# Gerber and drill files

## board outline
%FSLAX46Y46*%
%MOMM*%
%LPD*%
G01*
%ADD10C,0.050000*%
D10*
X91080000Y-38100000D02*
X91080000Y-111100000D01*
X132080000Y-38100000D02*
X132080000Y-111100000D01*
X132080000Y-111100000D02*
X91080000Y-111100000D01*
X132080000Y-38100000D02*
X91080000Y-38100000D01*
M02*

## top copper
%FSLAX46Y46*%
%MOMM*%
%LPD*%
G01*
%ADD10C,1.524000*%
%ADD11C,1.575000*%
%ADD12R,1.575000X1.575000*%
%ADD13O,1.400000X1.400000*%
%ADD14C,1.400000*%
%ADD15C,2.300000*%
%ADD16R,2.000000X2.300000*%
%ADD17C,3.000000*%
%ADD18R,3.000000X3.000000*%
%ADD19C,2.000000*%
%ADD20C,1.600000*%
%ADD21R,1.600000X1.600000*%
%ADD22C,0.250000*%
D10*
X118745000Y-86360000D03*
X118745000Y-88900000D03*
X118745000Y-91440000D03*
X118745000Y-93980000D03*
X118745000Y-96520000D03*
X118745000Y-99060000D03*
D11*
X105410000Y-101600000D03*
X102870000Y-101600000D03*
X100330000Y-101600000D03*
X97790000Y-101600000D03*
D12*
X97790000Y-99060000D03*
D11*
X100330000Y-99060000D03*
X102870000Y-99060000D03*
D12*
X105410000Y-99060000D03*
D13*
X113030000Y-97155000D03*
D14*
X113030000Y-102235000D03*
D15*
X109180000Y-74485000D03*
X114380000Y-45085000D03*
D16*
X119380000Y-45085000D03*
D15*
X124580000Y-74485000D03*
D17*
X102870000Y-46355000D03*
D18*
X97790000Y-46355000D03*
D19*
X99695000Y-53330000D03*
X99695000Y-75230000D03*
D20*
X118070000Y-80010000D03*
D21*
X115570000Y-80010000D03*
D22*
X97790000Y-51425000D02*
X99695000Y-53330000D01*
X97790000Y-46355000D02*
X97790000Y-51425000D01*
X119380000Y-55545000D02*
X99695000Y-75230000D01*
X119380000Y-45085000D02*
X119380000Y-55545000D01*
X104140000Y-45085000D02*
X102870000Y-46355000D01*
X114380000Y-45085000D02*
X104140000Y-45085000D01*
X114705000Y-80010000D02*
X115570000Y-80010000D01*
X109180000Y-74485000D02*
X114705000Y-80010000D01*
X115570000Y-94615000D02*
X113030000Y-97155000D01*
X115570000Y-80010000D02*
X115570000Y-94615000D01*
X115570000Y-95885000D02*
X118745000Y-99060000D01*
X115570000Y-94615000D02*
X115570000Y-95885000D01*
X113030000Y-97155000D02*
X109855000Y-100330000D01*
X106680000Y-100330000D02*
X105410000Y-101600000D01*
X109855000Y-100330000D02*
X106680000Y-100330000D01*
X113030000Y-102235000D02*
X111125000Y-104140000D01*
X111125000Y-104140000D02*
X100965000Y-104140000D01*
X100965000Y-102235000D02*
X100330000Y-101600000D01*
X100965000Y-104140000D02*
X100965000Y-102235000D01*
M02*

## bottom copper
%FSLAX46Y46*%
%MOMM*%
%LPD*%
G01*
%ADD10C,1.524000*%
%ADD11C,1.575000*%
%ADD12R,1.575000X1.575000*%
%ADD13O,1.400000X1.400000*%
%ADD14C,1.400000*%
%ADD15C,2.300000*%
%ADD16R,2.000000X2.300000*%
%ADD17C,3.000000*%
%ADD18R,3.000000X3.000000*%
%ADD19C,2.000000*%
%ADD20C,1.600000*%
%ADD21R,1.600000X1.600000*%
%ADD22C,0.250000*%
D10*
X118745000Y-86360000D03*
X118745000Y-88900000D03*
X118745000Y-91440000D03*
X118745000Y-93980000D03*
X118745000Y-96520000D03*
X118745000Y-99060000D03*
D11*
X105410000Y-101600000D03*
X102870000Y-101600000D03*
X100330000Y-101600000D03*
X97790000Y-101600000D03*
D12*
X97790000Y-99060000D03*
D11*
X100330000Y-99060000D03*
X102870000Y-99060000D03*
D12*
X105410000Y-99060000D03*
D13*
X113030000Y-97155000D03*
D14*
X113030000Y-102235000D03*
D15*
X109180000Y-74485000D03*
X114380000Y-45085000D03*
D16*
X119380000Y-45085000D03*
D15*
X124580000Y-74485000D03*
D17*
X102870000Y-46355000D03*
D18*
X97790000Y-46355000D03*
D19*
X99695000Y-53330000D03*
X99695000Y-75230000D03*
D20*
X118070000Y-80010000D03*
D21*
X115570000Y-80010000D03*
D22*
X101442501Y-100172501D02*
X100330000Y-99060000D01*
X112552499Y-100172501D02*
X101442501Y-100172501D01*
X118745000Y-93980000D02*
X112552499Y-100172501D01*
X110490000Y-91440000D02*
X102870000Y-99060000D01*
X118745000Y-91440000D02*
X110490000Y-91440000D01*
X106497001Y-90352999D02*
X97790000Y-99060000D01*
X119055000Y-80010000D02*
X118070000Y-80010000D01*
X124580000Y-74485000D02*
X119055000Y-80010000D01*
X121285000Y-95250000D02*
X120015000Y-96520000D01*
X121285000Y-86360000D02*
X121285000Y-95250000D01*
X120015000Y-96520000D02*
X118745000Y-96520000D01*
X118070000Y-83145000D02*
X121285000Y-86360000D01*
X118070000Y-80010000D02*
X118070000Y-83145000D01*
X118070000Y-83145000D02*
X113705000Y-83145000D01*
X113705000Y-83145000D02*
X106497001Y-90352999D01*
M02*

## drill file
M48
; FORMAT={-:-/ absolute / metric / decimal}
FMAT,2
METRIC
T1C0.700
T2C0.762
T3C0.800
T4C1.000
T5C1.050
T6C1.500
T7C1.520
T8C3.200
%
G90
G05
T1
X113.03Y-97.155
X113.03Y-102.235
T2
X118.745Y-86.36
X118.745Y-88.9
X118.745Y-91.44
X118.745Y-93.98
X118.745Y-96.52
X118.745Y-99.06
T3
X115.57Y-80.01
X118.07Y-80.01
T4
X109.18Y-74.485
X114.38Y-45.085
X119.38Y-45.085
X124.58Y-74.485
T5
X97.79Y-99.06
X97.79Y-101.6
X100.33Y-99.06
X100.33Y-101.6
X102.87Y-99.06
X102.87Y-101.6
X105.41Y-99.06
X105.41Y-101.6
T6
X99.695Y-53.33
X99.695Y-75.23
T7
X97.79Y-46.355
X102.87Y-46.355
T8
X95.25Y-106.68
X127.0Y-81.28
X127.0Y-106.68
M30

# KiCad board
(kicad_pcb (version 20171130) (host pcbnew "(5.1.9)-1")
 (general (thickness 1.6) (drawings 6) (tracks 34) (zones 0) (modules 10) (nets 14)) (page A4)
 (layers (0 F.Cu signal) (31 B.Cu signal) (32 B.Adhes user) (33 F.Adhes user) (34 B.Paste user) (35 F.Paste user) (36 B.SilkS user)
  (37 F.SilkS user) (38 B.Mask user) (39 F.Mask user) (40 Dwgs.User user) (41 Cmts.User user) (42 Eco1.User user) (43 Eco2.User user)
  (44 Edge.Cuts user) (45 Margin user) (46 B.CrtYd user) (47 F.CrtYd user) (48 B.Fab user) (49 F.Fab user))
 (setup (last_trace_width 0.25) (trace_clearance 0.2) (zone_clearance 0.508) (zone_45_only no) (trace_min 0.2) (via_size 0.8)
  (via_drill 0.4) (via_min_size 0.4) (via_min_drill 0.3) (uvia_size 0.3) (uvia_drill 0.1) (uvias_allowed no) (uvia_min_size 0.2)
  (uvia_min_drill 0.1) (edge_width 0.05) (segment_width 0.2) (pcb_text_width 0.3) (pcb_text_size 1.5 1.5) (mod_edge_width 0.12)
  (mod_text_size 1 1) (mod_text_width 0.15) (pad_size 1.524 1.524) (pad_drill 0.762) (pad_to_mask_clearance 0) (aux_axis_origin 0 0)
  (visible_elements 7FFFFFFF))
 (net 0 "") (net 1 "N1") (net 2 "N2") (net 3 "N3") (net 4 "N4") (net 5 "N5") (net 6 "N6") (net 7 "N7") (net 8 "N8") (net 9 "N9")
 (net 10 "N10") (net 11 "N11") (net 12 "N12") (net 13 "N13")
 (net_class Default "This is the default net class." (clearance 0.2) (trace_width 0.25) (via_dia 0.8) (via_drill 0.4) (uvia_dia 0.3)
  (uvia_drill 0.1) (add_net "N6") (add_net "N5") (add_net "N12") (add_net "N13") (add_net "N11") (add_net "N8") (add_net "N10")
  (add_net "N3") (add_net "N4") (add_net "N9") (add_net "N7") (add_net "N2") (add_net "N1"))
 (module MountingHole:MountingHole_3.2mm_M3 (layer F.Cu) (at 127 81.28)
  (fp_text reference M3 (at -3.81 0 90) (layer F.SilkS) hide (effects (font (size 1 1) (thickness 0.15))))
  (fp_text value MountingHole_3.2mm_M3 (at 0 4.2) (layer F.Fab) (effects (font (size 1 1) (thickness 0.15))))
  (pad 1 np_thru_hole circle (at 0 0) (size 3.2 3.2) (drill 3.2) (layers *.Cu *.Mask)))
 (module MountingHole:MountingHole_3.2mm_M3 (layer F.Cu) (at 127 106.68)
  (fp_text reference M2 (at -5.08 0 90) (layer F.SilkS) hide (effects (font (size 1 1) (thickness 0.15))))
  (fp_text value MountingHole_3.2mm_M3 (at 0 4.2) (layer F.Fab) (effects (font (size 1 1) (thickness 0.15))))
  (pad 1 np_thru_hole circle (at 0 0) (size 3.2 3.2) (drill 3.2) (layers *.Cu *.Mask)))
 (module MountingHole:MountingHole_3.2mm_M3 (layer F.Cu) (at 95.25 106.68)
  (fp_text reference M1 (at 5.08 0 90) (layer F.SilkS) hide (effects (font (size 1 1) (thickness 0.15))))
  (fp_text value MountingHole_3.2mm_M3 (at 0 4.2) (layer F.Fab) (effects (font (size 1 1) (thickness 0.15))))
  (pad 1 np_thru_hole circle (at 0 0) (size 3.2 3.2) (drill 3.2) (layers *.Cu *.Mask)))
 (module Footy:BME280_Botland (layer F.Cu) (at 127.635 100.33 180)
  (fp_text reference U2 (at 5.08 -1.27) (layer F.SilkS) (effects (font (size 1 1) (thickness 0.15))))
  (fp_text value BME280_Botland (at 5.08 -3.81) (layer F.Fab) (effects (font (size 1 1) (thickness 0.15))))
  (pad 6 thru_hole circle (at 8.89 13.97 180) (size 1.524 1.524) (drill 0.762) (layers *.Cu *.Mask) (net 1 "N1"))
  (pad 5 thru_hole circle (at 8.89 11.43 180) (size 1.524 1.524) (drill 0.762) (layers *.Cu *.Mask) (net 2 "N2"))
  (pad 4 thru_hole circle (at 8.89 8.89 180) (size 1.524 1.524) (drill 0.762) (layers *.Cu *.Mask) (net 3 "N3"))
  (pad 3 thru_hole circle (at 8.89 6.35 180) (size 1.524 1.524) (drill 0.762) (layers *.Cu *.Mask) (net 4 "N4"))
  (pad 2 thru_hole circle (at 8.89 3.81 180) (size 1.524 1.524) (drill 0.762) (layers *.Cu *.Mask) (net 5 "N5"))
  (pad 1 thru_hole circle (at 8.89 1.27 180) (size 1.524 1.524) (drill 0.762) (layers *.Cu *.Mask) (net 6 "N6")))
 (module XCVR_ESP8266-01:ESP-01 (layer F.Cu) (at 101.6 99.06 90)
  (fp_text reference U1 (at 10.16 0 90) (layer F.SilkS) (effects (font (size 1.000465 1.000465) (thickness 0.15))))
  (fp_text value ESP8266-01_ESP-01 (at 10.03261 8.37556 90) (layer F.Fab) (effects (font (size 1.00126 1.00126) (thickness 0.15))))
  (pad 8 thru_hole circle (at -2.54 3.81 90) (size 1.575 1.575) (drill 1.05) (layers *.Cu *.Mask) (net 6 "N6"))
  (pad 7 thru_hole circle (at -2.54 1.27 90) (size 1.575 1.575) (drill 1.05) (layers *.Cu *.Mask) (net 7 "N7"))
  (pad 6 thru_hole circle (at -2.54 -1.27 90) (size 1.575 1.575) (drill 1.05) (layers *.Cu *.Mask) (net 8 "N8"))
  (pad 5 thru_hole circle (at -2.54 -3.81 90) (size 1.575 1.575) (drill 1.05) (layers *.Cu *.Mask) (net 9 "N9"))
  (pad 4 thru_hole rect (at 0 -3.81 90) (size 1.575 1.575) (drill 1.05) (layers *.Cu *.Mask) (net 5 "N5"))
  (pad 3 thru_hole circle (at 0 -1.27 90) (size 1.575 1.575) (drill 1.05) (layers *.Cu *.Mask) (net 4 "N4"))
  (pad 2 thru_hole circle (at 0 1.27 90) (size 1.575 1.575) (drill 1.05) (layers *.Cu *.Mask) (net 3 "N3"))
  (pad 1 thru_hole rect (at 0 3.81 90) (size 1.575 1.575) (drill 1.05) (layers *.Cu *.Mask) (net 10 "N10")))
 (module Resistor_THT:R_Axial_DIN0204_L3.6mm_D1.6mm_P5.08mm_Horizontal (layer F.Cu) (at 113.03 102.235 90)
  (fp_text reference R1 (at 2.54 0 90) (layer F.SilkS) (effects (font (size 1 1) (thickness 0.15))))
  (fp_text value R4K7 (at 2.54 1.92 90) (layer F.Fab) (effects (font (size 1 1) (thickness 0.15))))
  (pad 2 thru_hole oval (at 5.08 0 90) (size 1.4 1.4) (drill 0.7) (layers *.Cu *.Mask) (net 6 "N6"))
  (pad 1 thru_hole circle (at 0 0 90) (size 1.4 1.4) (drill 0.7) (layers *.Cu *.Mask) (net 8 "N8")))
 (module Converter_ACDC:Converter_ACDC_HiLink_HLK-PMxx (layer F.Cu) (at 119.38 45.085 270)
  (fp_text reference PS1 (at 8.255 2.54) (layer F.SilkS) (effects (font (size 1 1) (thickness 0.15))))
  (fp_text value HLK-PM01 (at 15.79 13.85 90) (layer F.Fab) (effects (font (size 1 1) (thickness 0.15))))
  (pad 4 thru_hole circle (at 29.4 10.2 270) (size 2.3 2.3) (drill 1) (layers *.Cu *.Mask) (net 6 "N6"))
  (pad 2 thru_hole circle (at 0 5 270) (size 2.3 2.3) (drill 1) (layers *.Cu *.Mask) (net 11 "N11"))
  (pad 1 thru_hole rect (at 0 0 270) (size 2.3 2) (drill 1) (layers *.Cu *.Mask) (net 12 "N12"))
  (pad 3 thru_hole circle (at 29.4 -5.2 270) (size 2.3 2.3) (drill 1) (layers *.Cu *.Mask) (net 5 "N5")))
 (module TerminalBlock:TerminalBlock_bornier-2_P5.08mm (layer F.Cu) (at 97.79 46.355)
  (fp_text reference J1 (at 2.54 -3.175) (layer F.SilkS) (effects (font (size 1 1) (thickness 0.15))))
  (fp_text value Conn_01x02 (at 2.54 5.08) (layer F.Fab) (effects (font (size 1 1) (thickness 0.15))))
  (pad 2 thru_hole circle (at 5.08 0) (size 3 3) (drill 1.52) (layers *.Cu *.Mask) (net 11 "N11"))
  (pad 1 thru_hole rect (at 0 0) (size 3 3) (drill 1.52) (layers *.Cu *.Mask) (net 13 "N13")))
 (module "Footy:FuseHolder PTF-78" (layer F.Cu) (at 94.615 76.835 90)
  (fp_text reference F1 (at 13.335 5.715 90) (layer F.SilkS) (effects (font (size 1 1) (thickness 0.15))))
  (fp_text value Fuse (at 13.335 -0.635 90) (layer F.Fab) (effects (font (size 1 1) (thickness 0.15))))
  (pad 2 thru_hole circle (at 23.505 5.08 90) (size 2 2) (drill 1.5) (layers *.Cu *.Mask) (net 13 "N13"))
  (pad 1 thru_hole circle (at 1.605 5.08 90) (size 2 2) (drill 1.5) (layers *.Cu *.Mask) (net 12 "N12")))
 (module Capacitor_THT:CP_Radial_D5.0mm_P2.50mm (layer F.Cu) (at 115.57 80.01)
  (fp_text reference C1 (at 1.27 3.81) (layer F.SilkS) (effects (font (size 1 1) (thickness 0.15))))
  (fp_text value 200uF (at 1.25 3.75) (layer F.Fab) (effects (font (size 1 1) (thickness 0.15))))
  (pad 2 thru_hole circle (at 2.5 0) (size 1.6 1.6) (drill 0.8) (layers *.Cu *.Mask) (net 5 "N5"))
  (pad 1 thru_hole rect (at 0 0) (size 1.6 1.6) (drill 0.8) (layers *.Cu *.Mask) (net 6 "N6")))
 (gr_line (start 91.08 38.1) (end 91.08 111.1) (layer Edge.Cuts) (width 0.05))
 (gr_line (start 132.08 38.1) (end 132.08 111.1) (layer Edge.Cuts) (width 0.05))
 (gr_line (start 132.08 111.1) (end 91.08 111.1) (layer Edge.Cuts) (width 0.05))
 (gr_line (start 132.08 38.1) (end 91.08 38.1) (layer Edge.Cuts) (width 0.05))
 (segment (start 97.79 51.425) (end 99.695 53.33) (width 0.25) (layer F.Cu) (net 13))
 (segment (start 97.79 46.355) (end 97.79 51.425) (width 0.25) (layer F.Cu) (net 13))
 (segment (start 119.38 55.545) (end 99.695 75.23) (width 0.25) (layer F.Cu) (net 12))
 (segment (start 119.38 45.085) (end 119.38 55.545) (width 0.25) (layer F.Cu) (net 12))
 (segment (start 104.14 45.085) (end 102.87 46.355) (width 0.25) (layer F.Cu) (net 11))
 (segment (start 114.38 45.085) (end 104.14 45.085) (width 0.25) (layer F.Cu) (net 11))
 (segment (start 101.442501 100.172501) (end 100.33 99.06) (width 0.25) (layer B.Cu) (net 4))
 (segment (start 112.552499 100.172501) (end 101.442501 100.172501) (width 0.25) (layer B.Cu) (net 4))
 (segment (start 118.745 93.98) (end 112.552499 100.172501) (width 0.25) (layer B.Cu) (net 4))
 (segment (start 110.49 91.44) (end 102.87 99.06) (width 0.25) (layer B.Cu) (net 3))
 (segment (start 118.745 91.44) (end 110.49 91.44) (width 0.25) (layer B.Cu) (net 3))
 (segment (start 106.497001 90.352999) (end 97.79 99.06) (width 0.25) (layer B.Cu) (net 5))
 (segment (start 119.055 80.01) (end 118.07 80.01) (width 0.25) (layer B.Cu) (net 5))
 (segment (start 124.58 74.485) (end 119.055 80.01) (width 0.25) (layer B.Cu) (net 5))
 (segment (start 121.285 95.25) (end 120.015 96.52) (width 0.25) (layer B.Cu) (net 5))
 (segment (start 121.285 86.36) (end 121.285 95.25) (width 0.25) (layer B.Cu) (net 5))
 (segment (start 120.015 96.52) (end 118.745 96.52) (width 0.25) (layer B.Cu) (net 5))
 (segment (start 118.07 83.145) (end 121.285 86.36) (width 0.25) (layer B.Cu) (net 5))
 (segment (start 118.07 80.01) (end 118.07 83.145) (width 0.25) (layer B.Cu) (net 5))
 (segment (start 118.07 83.145) (end 113.705 83.145) (width 0.25) (layer B.Cu) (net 5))
 (segment (start 113.705 83.145) (end 106.497001 90.352999) (width 0.25) (layer B.Cu) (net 5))
 (segment (start 114.705 80.01) (end 115.57 80.01) (width 0.25) (layer F.Cu) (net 6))
 (segment (start 109.18 74.485) (end 114.705 80.01) (width 0.25) (layer F.Cu) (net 6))
 (segment (start 115.57 94.615) (end 113.03 97.155) (width 0.25) (layer F.Cu) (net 6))
 (segment (start 115.57 80.01) (end 115.57 94.615) (width 0.25) (layer F.Cu) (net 6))
 (segment (start 115.57 95.885) (end 118.745 99.06) (width 0.25) (layer F.Cu) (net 6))
 (segment (start 115.57 94.615) (end 115.57 95.885) (width 0.25) (layer F.Cu) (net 6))
 (segment (start 113.03 97.155) (end 109.855 100.33) (width 0.25) (layer F.Cu) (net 6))
 (segment (start 106.68 100.33) (end 105.41 101.6) (width 0.25) (layer F.Cu) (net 6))
 (segment (start 109.855 100.33) (end 106.68 100.33) (width 0.25) (layer F.Cu) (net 6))
 (segment (start 113.03 102.235) (end 111.125 104.14) (width 0.25) (layer F.Cu) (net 8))
 (segment (start 111.125 104.14) (end 100.965 104.14) (width 0.25) (layer F.Cu) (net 8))
 (segment (start 100.965 102.235) (end 100.33 101.6) (width 0.25) (layer F.Cu) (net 8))
 (segment (start 100.965 104.14) (end 100.965 102.235) (width 0.25) (layer F.Cu) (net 8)))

